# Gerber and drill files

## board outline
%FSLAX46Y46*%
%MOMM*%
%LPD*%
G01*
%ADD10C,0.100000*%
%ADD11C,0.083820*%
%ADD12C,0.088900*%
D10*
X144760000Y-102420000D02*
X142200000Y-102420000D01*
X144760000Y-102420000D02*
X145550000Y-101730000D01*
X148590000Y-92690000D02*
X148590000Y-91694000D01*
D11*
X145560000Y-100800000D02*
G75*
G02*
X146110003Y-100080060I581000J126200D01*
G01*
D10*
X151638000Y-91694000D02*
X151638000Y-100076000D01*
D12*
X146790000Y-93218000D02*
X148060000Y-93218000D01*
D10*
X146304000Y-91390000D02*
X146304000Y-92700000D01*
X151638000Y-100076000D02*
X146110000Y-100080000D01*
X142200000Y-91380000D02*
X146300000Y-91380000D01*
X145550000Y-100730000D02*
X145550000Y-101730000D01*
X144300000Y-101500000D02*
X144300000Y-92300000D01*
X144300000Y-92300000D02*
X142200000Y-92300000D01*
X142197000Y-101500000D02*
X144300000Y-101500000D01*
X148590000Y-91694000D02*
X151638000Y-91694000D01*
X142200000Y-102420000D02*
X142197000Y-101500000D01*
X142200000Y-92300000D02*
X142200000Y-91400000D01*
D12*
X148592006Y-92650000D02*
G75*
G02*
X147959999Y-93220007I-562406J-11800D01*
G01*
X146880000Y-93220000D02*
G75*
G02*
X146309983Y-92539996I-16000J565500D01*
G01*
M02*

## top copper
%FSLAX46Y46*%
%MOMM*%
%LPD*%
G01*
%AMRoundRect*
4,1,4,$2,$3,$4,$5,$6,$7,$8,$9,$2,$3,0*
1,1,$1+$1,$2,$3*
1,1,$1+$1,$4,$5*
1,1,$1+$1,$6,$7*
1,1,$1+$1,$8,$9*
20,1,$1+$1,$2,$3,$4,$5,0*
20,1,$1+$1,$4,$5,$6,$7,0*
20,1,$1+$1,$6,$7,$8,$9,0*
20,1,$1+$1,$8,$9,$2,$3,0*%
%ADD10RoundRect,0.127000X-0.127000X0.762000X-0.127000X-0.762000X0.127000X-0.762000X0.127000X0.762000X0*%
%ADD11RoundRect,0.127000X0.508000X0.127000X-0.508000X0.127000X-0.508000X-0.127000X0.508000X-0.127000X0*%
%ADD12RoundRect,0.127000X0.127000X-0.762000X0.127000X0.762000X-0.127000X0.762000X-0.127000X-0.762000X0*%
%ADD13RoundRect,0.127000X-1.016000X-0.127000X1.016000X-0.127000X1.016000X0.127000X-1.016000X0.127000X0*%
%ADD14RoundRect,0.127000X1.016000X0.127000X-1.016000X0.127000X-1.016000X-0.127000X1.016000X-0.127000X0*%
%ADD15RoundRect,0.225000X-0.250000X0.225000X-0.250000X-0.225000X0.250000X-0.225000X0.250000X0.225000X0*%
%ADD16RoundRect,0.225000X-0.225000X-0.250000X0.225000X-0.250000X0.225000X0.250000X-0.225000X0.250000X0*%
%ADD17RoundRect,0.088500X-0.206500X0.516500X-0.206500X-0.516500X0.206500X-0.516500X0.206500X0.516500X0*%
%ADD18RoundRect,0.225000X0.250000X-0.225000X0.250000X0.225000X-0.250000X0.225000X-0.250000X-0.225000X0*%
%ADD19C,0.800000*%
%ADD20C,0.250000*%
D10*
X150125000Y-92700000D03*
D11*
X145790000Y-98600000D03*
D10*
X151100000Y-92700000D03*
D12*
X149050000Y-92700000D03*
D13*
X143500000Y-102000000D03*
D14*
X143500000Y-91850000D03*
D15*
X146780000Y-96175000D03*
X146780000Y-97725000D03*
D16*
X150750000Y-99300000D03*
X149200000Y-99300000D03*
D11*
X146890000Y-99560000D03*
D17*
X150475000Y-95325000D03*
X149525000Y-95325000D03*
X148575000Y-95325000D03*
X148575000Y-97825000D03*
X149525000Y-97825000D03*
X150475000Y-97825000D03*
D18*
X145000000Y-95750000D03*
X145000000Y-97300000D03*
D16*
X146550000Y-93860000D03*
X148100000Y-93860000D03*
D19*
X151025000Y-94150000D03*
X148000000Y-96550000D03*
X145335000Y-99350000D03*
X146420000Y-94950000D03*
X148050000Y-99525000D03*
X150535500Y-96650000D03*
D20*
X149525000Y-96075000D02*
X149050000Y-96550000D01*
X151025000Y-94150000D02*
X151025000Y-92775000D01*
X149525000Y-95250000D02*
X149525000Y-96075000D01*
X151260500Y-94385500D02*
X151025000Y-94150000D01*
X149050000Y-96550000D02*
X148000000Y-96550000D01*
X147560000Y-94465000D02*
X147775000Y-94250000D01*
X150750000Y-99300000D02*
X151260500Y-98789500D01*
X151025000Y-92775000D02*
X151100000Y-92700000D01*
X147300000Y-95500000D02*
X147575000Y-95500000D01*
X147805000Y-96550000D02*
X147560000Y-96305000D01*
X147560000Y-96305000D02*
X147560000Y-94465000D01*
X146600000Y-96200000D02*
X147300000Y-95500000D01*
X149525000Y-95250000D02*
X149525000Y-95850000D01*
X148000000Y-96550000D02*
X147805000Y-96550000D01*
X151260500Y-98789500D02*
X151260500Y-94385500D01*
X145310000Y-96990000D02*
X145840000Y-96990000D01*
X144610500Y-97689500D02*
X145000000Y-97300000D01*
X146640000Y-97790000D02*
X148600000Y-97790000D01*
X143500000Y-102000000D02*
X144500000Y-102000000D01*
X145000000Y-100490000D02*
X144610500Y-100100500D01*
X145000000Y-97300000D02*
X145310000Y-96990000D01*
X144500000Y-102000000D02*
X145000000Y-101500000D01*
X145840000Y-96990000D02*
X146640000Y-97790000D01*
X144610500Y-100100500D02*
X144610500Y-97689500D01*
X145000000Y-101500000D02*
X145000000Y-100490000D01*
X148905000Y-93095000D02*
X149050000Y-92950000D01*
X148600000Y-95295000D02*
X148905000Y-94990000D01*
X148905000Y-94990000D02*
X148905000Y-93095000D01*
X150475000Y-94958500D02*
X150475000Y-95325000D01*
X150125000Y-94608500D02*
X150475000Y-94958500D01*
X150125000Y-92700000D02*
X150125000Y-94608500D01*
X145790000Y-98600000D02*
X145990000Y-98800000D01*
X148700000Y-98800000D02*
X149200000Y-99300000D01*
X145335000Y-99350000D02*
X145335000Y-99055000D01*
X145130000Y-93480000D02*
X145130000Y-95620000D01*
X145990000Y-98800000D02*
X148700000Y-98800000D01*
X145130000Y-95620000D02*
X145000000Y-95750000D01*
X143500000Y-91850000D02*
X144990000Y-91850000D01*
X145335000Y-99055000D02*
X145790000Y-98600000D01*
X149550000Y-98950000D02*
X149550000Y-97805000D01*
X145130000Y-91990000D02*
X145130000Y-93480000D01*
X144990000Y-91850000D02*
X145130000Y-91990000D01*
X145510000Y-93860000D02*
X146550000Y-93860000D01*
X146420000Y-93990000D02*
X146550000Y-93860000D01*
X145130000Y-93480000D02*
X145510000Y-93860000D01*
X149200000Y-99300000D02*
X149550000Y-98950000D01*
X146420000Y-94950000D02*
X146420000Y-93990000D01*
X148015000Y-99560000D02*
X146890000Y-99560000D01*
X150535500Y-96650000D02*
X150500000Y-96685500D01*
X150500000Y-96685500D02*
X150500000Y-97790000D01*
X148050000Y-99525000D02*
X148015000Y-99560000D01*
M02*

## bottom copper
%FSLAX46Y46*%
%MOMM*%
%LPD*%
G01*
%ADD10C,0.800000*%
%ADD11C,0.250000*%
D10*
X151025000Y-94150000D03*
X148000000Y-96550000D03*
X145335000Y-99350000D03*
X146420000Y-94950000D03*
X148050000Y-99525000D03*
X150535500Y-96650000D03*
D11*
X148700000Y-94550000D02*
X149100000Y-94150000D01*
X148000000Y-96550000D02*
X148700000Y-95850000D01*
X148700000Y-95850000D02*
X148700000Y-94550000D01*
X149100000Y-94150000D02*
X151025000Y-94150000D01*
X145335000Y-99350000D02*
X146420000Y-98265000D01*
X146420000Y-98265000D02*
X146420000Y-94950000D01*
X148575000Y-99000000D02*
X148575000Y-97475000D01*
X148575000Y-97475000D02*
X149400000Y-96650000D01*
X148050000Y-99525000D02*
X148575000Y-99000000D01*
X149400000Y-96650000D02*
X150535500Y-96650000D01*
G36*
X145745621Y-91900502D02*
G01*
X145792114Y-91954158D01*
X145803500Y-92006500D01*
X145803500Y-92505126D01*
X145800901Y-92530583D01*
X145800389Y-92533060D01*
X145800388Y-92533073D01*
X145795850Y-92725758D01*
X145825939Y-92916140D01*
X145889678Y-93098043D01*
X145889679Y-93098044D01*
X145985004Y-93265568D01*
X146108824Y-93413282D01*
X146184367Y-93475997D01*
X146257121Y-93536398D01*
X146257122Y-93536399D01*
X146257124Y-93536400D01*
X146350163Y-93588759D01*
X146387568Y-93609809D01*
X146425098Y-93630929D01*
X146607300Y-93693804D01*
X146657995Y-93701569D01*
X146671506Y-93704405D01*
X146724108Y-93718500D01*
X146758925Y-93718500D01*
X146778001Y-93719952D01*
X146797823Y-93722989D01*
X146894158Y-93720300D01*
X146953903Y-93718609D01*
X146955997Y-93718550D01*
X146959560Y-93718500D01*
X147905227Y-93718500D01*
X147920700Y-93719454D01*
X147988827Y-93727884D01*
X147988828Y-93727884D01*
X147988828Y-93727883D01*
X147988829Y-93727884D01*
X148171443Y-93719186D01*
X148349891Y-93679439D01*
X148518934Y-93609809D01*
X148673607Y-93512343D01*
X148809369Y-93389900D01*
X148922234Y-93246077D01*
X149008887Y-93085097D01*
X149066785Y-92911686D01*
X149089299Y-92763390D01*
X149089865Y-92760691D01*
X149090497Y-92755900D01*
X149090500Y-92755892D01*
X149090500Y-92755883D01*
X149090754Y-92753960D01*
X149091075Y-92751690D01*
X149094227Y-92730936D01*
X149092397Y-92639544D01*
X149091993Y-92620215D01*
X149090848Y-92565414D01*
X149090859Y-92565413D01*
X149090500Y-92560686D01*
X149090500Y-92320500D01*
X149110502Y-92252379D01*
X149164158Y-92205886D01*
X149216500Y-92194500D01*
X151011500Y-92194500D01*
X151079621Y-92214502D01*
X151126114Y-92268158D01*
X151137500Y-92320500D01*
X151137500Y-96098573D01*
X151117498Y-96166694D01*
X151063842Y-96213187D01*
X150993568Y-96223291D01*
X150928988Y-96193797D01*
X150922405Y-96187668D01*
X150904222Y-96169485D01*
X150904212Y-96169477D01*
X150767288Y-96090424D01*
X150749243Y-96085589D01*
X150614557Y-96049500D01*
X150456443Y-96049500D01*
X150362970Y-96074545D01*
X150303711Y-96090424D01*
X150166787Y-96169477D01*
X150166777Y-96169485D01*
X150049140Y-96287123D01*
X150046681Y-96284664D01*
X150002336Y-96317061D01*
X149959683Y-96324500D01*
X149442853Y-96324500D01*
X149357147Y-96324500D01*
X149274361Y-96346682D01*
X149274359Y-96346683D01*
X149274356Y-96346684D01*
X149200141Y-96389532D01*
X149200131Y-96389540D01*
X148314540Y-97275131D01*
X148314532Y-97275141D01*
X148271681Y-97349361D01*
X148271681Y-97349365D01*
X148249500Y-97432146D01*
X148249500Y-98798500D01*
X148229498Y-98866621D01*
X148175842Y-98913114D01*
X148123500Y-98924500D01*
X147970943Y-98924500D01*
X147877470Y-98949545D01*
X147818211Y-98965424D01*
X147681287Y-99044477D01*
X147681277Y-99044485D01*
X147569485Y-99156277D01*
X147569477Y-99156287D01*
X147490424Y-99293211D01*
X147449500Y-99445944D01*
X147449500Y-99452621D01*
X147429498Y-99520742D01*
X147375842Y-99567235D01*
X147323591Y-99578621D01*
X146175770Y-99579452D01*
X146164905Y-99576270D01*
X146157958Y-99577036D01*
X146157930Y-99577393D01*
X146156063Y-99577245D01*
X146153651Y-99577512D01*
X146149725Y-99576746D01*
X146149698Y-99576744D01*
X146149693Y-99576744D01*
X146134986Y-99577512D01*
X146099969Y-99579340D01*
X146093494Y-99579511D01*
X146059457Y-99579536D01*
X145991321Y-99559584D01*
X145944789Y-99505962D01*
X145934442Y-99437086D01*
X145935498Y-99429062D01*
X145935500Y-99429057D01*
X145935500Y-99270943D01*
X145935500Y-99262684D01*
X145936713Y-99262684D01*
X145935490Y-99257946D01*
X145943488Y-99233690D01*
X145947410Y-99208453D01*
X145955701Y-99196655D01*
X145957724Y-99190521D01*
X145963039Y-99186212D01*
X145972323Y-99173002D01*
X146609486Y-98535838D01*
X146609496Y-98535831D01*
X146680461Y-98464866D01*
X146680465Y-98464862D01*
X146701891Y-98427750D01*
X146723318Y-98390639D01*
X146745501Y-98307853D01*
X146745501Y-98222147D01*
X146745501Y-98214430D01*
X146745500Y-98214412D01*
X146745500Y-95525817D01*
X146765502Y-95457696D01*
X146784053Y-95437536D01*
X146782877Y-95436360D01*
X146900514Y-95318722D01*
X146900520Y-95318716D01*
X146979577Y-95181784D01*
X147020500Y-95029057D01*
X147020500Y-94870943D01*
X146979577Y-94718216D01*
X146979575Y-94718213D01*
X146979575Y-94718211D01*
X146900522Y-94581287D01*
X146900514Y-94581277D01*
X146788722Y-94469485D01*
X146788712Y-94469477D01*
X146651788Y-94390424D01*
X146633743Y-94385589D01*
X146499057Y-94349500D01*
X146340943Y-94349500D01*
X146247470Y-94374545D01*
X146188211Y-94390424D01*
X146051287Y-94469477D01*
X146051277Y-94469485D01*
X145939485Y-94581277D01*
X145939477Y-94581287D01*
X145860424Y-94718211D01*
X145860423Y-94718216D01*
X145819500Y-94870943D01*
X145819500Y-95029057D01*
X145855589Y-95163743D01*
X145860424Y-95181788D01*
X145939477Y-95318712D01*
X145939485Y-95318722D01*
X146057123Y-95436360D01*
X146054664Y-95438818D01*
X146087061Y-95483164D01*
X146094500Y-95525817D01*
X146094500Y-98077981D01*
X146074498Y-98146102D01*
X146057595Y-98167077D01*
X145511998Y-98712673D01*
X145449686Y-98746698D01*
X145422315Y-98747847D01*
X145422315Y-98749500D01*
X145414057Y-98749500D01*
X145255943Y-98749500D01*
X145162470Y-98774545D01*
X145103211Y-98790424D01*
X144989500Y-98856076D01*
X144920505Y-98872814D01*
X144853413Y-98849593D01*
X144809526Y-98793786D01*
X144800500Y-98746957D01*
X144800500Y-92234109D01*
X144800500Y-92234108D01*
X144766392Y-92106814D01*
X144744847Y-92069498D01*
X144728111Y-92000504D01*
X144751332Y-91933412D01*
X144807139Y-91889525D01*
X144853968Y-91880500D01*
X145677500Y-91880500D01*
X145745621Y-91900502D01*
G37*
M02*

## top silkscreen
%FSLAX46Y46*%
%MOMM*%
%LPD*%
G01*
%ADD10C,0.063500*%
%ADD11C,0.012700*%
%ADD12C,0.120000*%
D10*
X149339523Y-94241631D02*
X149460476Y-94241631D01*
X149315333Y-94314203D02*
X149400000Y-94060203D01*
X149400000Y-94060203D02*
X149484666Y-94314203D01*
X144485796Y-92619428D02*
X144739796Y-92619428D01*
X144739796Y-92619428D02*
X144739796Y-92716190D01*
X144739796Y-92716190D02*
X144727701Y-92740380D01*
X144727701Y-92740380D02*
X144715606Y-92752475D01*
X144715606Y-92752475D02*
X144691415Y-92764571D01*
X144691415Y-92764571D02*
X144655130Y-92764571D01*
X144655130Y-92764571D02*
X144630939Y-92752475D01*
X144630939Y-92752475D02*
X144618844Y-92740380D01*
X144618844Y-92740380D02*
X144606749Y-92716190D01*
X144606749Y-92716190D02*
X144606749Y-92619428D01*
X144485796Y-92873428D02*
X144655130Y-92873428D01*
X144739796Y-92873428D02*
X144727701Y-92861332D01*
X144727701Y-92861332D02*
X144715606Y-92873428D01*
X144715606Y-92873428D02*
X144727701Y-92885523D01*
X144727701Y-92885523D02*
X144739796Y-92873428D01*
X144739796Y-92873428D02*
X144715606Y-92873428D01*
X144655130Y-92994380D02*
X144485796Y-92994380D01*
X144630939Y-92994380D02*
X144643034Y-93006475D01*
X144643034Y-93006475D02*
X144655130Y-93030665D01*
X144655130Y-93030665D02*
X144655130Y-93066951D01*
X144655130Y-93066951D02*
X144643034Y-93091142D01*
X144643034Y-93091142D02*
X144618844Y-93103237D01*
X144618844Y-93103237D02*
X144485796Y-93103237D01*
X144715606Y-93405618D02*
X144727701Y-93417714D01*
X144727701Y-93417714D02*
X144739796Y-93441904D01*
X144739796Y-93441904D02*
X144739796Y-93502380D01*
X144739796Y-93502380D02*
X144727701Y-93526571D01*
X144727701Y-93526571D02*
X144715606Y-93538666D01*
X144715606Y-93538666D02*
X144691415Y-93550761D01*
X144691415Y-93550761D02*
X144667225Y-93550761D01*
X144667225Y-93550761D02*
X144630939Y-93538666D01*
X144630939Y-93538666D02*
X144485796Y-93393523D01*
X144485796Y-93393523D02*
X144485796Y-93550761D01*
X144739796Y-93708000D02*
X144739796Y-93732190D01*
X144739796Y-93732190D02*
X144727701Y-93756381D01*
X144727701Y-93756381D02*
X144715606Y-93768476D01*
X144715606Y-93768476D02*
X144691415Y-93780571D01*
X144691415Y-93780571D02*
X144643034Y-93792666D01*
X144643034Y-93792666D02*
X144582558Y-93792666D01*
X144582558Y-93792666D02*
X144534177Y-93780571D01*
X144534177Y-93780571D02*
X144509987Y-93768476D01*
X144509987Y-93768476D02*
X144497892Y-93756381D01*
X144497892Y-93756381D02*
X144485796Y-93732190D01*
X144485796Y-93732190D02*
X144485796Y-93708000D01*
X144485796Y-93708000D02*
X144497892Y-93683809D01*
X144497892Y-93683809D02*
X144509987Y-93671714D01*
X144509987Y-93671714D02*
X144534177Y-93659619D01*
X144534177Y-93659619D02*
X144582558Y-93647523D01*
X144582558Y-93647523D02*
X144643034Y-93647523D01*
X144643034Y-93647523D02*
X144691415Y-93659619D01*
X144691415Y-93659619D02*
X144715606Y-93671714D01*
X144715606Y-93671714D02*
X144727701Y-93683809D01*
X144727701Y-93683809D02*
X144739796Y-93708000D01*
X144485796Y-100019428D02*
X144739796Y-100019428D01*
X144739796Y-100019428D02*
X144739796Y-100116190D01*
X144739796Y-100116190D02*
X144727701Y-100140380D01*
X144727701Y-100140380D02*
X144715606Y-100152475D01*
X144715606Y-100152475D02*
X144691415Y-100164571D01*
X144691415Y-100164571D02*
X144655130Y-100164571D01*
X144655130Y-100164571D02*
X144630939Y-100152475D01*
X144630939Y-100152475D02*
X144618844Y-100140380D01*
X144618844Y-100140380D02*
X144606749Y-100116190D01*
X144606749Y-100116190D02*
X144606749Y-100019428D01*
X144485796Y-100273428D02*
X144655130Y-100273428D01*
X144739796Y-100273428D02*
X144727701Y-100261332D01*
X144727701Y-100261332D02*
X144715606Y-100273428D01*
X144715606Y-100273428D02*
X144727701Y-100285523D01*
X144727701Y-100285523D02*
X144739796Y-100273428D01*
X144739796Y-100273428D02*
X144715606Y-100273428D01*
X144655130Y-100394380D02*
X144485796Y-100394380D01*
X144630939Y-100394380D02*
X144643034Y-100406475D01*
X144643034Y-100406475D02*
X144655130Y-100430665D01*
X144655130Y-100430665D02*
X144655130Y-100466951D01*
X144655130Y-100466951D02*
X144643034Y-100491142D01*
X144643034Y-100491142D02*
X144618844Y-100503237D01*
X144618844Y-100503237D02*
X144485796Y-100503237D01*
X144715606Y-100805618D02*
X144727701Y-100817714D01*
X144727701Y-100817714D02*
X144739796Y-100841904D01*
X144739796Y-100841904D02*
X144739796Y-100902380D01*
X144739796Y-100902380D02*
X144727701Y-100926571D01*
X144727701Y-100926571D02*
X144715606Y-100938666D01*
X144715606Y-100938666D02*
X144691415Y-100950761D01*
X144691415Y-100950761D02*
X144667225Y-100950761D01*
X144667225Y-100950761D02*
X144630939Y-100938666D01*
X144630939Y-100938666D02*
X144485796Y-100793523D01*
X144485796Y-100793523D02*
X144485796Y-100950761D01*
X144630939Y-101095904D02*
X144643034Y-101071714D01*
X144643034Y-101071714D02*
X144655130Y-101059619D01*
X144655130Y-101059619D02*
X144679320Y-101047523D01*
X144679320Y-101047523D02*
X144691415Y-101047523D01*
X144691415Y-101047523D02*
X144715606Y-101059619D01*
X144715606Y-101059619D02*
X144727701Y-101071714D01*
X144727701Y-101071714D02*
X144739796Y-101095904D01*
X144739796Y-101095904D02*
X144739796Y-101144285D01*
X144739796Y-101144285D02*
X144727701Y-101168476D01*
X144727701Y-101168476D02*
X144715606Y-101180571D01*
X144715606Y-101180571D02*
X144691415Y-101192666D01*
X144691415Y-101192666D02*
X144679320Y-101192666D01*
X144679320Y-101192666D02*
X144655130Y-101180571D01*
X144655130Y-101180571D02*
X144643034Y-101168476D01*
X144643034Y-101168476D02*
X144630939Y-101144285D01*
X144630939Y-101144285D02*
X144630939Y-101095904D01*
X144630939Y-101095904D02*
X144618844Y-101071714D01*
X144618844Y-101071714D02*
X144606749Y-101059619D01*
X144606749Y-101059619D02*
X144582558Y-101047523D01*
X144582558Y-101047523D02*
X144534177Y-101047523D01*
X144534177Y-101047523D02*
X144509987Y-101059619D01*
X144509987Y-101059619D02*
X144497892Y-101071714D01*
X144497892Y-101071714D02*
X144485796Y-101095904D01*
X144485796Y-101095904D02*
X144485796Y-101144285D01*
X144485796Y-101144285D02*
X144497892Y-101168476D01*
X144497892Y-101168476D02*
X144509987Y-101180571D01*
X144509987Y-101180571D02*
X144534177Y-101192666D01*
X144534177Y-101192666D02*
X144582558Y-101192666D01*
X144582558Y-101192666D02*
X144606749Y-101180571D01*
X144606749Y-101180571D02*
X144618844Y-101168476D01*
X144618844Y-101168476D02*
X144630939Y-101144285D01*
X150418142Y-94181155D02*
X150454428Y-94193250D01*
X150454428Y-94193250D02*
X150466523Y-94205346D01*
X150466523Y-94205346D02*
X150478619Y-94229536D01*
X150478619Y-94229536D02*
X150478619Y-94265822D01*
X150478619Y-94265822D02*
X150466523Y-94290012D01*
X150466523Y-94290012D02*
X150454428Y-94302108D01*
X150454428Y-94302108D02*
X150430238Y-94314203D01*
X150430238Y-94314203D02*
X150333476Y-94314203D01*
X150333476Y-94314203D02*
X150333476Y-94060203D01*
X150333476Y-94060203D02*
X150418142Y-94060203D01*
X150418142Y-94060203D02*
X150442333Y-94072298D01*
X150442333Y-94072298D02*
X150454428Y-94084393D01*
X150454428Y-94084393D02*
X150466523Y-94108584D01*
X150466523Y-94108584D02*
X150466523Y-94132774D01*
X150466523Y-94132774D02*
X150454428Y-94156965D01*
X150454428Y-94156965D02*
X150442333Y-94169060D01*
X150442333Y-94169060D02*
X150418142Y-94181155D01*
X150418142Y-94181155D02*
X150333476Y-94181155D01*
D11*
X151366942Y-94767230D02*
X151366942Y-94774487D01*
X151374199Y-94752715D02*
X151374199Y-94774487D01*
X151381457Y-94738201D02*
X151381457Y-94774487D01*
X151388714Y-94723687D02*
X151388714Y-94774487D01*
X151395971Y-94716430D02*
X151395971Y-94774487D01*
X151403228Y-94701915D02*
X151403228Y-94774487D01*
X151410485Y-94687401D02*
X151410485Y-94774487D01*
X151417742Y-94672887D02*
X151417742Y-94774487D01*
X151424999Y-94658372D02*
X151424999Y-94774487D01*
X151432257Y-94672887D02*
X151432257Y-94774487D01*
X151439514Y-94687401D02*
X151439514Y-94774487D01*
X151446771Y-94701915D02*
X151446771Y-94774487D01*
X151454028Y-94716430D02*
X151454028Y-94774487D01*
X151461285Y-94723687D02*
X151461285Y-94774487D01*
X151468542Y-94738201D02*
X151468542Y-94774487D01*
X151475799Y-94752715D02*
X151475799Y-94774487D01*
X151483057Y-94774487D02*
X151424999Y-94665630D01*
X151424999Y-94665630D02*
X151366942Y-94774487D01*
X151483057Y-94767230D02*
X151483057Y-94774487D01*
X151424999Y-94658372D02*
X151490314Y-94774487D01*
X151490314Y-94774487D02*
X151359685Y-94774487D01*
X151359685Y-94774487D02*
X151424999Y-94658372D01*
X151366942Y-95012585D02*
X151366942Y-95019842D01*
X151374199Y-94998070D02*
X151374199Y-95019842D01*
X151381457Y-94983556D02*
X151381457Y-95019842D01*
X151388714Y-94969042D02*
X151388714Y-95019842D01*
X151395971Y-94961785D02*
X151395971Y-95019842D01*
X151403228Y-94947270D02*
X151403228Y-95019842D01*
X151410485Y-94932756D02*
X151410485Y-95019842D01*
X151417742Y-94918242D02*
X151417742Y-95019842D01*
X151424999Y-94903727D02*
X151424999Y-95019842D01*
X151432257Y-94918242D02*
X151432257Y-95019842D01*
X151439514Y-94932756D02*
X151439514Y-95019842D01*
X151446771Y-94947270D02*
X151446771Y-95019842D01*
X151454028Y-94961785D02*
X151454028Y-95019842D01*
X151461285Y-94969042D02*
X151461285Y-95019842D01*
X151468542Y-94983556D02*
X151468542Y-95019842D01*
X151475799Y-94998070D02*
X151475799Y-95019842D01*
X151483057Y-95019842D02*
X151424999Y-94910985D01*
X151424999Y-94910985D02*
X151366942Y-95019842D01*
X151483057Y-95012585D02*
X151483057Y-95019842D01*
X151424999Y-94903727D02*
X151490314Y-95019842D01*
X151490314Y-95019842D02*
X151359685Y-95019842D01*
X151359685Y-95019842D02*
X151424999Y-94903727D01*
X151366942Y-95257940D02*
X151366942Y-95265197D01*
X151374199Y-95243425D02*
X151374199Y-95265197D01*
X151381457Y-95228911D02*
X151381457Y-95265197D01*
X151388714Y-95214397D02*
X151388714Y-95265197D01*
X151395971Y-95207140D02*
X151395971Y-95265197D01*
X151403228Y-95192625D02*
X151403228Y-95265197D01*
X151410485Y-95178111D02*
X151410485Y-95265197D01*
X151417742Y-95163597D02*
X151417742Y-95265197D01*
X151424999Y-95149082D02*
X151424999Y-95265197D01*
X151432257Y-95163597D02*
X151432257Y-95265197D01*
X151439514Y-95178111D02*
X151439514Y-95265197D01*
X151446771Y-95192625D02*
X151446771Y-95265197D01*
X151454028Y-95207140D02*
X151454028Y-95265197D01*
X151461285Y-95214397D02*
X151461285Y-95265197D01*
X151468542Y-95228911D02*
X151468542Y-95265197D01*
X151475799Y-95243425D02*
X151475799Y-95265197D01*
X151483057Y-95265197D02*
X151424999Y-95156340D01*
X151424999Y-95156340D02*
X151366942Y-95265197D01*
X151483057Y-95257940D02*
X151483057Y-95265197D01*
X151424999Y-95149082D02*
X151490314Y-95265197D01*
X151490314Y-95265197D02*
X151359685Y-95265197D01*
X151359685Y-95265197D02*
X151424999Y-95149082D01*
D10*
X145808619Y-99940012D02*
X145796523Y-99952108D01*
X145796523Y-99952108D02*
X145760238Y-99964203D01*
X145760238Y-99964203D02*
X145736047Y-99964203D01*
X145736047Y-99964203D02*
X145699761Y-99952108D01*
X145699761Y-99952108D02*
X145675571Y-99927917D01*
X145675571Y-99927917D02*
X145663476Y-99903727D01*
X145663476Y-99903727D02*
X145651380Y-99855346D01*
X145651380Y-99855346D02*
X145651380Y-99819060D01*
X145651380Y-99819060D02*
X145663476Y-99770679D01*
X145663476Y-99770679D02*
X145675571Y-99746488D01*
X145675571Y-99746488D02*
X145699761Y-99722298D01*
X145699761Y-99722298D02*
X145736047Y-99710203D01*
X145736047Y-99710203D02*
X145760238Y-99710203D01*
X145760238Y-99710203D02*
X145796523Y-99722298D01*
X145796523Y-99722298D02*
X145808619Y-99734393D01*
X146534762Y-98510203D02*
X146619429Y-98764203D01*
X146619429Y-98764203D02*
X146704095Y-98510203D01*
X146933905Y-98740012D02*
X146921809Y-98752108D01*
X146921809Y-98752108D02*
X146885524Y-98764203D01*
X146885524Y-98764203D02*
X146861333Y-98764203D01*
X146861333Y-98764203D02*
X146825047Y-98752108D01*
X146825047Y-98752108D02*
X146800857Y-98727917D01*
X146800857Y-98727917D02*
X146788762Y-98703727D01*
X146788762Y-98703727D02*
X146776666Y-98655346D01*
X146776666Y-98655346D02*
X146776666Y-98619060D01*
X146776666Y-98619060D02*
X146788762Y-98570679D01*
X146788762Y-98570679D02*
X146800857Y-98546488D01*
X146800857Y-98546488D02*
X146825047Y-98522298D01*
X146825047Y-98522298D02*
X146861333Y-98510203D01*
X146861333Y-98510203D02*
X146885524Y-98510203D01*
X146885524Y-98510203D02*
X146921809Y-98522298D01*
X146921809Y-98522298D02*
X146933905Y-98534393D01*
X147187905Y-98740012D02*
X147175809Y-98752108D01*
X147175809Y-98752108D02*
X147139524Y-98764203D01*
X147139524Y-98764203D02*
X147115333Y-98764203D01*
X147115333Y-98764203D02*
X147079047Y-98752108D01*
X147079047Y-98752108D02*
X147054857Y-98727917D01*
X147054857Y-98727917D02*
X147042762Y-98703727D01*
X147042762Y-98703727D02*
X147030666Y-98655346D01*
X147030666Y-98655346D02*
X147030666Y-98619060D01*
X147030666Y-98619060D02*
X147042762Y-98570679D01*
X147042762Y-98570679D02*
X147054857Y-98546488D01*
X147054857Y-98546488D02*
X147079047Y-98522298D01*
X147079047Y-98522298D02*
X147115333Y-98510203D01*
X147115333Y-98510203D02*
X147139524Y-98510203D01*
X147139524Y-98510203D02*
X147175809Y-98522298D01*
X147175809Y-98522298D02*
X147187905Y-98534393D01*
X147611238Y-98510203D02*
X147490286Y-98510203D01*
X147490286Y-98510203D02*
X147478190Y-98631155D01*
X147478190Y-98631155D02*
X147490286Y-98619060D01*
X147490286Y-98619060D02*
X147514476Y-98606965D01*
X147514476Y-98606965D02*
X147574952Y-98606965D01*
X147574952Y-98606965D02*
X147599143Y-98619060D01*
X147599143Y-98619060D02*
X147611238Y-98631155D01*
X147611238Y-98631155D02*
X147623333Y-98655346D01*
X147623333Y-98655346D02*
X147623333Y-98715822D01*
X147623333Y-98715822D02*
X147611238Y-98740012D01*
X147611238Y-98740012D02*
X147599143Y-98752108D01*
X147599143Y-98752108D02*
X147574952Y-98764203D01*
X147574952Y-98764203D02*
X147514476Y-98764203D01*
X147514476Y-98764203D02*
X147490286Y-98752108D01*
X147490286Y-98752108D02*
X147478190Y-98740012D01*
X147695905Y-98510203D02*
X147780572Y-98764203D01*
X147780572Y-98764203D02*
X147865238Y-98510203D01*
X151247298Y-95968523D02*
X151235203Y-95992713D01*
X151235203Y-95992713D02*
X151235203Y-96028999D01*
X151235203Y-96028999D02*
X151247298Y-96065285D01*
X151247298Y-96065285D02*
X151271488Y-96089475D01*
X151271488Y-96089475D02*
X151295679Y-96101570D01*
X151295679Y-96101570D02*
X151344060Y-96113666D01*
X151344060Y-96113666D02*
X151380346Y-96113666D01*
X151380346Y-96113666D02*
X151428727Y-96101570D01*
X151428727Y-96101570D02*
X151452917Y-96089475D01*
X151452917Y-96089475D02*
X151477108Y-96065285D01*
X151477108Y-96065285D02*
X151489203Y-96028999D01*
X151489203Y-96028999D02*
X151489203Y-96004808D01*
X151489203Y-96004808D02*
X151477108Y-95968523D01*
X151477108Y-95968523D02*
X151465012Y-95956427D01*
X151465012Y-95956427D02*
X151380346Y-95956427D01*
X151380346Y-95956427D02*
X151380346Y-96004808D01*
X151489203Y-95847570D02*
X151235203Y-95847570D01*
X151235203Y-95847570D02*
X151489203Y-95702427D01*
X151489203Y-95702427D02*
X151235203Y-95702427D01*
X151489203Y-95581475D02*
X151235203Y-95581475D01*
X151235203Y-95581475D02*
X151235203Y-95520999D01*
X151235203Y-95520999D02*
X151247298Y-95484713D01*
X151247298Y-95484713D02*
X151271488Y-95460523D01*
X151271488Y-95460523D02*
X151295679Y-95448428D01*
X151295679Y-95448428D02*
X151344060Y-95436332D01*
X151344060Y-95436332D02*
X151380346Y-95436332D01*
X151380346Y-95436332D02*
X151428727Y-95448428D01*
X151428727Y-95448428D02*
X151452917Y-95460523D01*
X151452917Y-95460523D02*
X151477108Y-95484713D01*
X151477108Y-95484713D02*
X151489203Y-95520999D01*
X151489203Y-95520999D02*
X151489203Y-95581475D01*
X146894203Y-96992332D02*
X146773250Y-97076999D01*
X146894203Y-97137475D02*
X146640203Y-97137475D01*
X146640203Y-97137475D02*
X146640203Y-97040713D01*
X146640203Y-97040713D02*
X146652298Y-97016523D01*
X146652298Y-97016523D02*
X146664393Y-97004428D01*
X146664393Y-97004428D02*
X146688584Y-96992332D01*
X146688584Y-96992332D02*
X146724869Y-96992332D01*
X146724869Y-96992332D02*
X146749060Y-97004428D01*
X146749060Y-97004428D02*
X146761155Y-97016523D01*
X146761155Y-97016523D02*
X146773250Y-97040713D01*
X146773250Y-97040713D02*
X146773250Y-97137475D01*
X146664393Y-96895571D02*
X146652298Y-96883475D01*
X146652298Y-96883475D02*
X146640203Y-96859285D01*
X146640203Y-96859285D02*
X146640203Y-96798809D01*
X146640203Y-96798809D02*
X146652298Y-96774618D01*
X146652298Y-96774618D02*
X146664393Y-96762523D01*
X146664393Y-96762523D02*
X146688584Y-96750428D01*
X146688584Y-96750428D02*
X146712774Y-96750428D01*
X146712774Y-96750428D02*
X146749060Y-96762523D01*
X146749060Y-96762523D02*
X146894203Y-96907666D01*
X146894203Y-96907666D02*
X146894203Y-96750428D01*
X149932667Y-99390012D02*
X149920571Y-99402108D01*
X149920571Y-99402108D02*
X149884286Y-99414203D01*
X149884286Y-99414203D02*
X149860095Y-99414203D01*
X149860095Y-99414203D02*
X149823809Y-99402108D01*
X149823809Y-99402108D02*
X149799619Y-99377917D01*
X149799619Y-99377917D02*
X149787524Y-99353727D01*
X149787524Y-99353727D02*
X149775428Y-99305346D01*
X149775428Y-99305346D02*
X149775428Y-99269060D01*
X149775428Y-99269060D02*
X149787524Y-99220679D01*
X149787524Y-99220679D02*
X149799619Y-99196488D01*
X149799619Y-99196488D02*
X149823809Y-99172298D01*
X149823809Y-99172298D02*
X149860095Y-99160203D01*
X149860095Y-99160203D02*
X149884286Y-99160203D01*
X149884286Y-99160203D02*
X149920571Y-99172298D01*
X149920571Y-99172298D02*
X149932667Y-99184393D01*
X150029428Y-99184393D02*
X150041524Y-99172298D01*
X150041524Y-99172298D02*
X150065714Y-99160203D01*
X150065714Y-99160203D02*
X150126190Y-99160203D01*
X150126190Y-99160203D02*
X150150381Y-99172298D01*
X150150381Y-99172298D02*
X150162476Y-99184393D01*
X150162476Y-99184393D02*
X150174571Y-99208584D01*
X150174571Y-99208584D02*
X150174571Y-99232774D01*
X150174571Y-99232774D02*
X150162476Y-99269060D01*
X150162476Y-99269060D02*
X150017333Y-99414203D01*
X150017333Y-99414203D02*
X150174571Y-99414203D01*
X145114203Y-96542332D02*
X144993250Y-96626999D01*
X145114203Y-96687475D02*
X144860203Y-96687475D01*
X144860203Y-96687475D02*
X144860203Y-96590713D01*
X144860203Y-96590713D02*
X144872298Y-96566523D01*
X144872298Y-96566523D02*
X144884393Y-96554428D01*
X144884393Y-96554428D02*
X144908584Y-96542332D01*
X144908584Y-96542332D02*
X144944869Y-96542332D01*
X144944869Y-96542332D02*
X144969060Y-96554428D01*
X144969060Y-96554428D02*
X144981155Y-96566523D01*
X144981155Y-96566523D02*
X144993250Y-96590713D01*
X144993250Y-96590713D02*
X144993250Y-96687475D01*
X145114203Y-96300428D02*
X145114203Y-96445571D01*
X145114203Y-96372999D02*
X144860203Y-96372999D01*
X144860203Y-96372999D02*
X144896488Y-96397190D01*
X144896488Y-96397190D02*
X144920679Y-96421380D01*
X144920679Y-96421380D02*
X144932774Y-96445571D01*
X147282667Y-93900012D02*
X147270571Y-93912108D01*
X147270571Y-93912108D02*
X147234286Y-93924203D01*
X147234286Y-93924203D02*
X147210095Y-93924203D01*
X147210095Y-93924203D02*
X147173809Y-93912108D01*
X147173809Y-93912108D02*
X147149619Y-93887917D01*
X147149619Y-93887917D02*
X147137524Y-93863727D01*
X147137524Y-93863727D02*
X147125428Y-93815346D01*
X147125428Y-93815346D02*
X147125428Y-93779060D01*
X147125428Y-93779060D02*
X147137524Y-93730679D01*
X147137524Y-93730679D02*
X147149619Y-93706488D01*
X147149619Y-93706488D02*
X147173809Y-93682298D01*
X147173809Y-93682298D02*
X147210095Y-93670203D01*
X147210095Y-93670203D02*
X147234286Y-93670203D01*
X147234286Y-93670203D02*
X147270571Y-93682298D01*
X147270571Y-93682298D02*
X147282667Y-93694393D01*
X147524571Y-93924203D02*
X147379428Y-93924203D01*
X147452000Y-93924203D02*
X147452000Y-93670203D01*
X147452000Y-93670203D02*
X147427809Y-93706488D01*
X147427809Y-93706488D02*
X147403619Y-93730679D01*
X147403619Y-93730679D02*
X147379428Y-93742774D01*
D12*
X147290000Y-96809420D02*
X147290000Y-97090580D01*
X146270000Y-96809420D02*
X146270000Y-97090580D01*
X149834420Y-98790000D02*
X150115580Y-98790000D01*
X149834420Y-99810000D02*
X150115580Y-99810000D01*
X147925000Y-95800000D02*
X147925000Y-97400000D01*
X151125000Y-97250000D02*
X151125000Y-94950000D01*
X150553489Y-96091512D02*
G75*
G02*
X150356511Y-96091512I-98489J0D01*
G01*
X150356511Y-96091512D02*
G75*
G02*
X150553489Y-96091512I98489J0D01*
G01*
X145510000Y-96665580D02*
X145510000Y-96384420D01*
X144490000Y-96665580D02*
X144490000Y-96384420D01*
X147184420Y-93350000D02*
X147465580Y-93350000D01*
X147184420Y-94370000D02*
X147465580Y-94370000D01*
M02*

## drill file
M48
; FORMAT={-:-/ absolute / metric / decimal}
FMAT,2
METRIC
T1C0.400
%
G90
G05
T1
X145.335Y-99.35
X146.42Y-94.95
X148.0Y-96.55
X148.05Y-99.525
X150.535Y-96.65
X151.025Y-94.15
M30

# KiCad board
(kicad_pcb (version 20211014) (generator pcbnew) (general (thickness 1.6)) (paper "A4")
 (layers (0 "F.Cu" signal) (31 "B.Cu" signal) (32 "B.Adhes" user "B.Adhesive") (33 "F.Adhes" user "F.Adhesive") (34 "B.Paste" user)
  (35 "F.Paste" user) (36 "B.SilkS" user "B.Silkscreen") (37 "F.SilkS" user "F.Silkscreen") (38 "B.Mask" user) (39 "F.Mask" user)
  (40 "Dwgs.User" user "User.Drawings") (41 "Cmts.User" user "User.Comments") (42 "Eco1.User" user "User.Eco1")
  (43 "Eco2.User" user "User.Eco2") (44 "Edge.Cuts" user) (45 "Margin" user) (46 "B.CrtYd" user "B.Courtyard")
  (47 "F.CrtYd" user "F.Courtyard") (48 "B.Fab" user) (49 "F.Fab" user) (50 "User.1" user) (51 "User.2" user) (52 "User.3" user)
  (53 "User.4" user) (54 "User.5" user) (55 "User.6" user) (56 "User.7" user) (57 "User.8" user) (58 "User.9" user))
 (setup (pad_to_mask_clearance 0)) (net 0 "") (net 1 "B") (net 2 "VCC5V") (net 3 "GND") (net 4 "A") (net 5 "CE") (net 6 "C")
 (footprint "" (layer "F.Cu") (at 150.125 92.7 90)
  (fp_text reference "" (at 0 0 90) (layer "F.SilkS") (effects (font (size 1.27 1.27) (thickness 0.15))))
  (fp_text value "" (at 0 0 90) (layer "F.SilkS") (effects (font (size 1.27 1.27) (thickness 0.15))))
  (pad "10" smd roundrect (at 0 0 270) (size 1.778 0.508) (layers "F.Cu" "F.Paste" "F.Mask") (roundrect_rratio 0.25) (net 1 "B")))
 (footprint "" (layer "F.Cu") (at 145.79 98.6 -90)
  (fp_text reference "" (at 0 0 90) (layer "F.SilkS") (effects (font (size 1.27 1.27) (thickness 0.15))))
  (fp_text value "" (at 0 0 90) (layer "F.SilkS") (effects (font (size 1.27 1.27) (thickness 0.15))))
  (pad "B" smd roundrect (at 0 0 180) (size 1.27 0.508) (layers "F.Cu" "F.Paste" "F.Mask") (roundrect_rratio 0.25) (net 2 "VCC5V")))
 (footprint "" (layer "F.Cu") (at 151.1 92.7 90)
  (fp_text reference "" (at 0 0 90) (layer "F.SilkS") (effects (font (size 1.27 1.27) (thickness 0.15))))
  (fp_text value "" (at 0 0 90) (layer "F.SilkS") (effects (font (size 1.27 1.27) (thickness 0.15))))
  (pad "9" smd roundrect (at 0 0 270) (size 1.778 0.508) (layers "F.Cu" "F.Paste" "F.Mask") (roundrect_rratio 0.25) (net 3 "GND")))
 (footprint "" (layer "F.Cu") (at 149.05 92.7 -90)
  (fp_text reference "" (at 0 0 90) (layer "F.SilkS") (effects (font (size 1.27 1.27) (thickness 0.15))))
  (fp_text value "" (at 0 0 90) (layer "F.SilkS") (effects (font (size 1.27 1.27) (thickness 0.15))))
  (pad "11" smd roundrect (at 0 0 90) (size 1.778 0.508) (layers "F.Cu" "F.Paste" "F.Mask") (roundrect_rratio 0.25) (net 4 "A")))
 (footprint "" (layer "F.Cu") (at 143.5 102)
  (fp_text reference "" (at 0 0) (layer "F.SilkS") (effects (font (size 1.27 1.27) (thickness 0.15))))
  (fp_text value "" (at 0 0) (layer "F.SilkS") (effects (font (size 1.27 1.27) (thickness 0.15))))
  (pad "4" smd roundrect (at 0 0) (size 2.286 0.508) (layers "F.Cu" "F.Paste" "F.Mask") (roundrect_rratio 0.25) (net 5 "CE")))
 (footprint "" (layer "F.Cu") (at 143.5 91.85 180)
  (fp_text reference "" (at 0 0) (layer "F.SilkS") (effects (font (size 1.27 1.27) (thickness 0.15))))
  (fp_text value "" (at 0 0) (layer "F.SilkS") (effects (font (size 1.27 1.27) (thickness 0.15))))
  (pad "1" smd roundrect (at 0 0 180) (size 2.286 0.508) (layers "F.Cu" "F.Paste" "F.Mask") (roundrect_rratio 0.25) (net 2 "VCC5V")))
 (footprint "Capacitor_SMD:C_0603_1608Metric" (layer "F.Cu") (at 146.78 96.95 -90)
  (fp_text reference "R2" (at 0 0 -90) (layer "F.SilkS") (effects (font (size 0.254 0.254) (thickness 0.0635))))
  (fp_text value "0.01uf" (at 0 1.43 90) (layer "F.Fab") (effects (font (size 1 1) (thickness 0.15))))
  (fp_line (start -0.14058 -0.51) (end 0.14058 -0.51) (layer "F.SilkS") (width 0.12))
  (fp_line (start -0.14058 0.51) (end 0.14058 0.51) (layer "F.SilkS") (width 0.12))
  (pad "5" smd roundrect (at -0.775 0 270) (size 0.9 0.95) (layers "F.Cu" "F.Paste" "F.Mask") (roundrect_rratio 0.25) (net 3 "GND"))
  (pad "6" smd roundrect (at 0.775 0 270) (size 0.9 0.95) (layers "F.Cu" "F.Paste" "F.Mask") (roundrect_rratio 0.25) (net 5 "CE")))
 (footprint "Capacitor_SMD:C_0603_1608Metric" (layer "F.Cu") (at 149.975 99.3)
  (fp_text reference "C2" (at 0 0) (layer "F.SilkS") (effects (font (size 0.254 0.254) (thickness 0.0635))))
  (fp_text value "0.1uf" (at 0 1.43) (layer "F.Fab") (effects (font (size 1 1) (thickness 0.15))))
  (fp_line (start -0.14058 -0.51) (end 0.14058 -0.51) (layer "F.SilkS") (width 0.12))
  (fp_line (start -0.14058 0.51) (end 0.14058 0.51) (layer "F.SilkS") (width 0.12))
  (pad "7" smd roundrect (at 0.775 0) (size 0.9 0.95) (layers "F.Cu" "F.Paste" "F.Mask") (roundrect_rratio 0.25) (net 3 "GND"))
  (pad "8" smd roundrect (at -0.775 0) (size 0.9 0.95) (layers "F.Cu" "F.Paste" "F.Mask") (roundrect_rratio 0.25) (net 2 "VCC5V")))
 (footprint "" (layer "F.Cu") (at 146.89 99.56)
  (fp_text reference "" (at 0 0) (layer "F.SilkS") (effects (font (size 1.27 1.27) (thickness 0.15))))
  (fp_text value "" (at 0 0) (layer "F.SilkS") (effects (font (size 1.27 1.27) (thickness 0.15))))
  (pad "B" smd roundrect (at 0 0 180) (size 1.27 0.508) (layers "F.Cu" "F.Paste" "F.Mask") (roundrect_rratio 0.25) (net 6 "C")))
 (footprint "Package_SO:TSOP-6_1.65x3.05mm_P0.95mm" (layer "F.Cu") (at 149.525 96.45 -90)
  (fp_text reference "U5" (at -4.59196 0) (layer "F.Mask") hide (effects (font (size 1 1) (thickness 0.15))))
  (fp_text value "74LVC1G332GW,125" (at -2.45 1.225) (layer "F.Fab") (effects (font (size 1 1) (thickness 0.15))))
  (fp_line (start -0.65 1.6) (end 0.95 1.6) (layer "F.SilkS") (width 0.12))
  (fp_line (start 0.8 -1.6) (end -1.5 -1.6) (layer "F.SilkS") (width 0.12))
  (fp_circle (center -0.358488 -0.93) (end -0.268488 -0.89) (layer "F.SilkS") (width 0.12) (fill none))
  (pad "1" smd roundrect (at -1.125 -0.95 270) (size 1.21 0.59) (layers "F.Cu" "F.Paste" "F.Mask") (roundrect_rratio 0.15) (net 1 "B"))
  (pad "2" smd roundrect (at -1.125 0 270) (size 1.21 0.59) (layers "F.Cu" "F.Paste" "F.Mask") (roundrect_rratio 0.15) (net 3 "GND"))
  (pad "3" smd roundrect (at -1.125 0.95 270) (size 1.21 0.59) (layers "F.Cu" "F.Paste" "F.Mask") (roundrect_rratio 0.15) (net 4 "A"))
  (pad "4" smd roundrect (at 1.375 0.95 270) (size 1.21 0.59) (layers "F.Cu" "F.Paste" "F.Mask") (roundrect_rratio 0.15) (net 5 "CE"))
  (pad "5" smd roundrect (at 1.375 0 270) (size 1.21 0.59) (layers "F.Cu" "F.Paste" "F.Mask") (roundrect_rratio 0.15) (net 2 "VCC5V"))
  (pad "6" smd roundrect (at 1.375 -0.95 270) (size 1.21 0.59) (layers "F.Cu" "F.Paste" "F.Mask") (roundrect_rratio 0.15) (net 6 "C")))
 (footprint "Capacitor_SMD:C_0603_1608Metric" (layer "F.Cu") (at 145 96.525 90)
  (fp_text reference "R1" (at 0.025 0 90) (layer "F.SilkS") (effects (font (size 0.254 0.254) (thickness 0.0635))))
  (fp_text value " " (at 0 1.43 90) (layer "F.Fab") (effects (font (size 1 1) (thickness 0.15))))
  (fp_line (start -0.14058 0.51) (end 0.14058 0.51) (layer "F.SilkS") (width 0.12))
  (fp_line (start -0.14058 -0.51) (end 0.14058 -0.51) (layer "F.SilkS") (width 0.12))
  (pad "2" smd roundrect (at 0.775 0 90) (size 0.9 0.95) (layers "F.Cu" "F.Paste" "F.Mask") (roundrect_rratio 0.25) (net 2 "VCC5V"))
  (pad "3" smd roundrect (at -0.775 0 90) (size 0.9 0.95) (layers "F.Cu" "F.Paste" "F.Mask") (roundrect_rratio 0.25) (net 5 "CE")))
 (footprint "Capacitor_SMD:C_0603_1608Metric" (layer "F.Cu") (at 147.325 93.86)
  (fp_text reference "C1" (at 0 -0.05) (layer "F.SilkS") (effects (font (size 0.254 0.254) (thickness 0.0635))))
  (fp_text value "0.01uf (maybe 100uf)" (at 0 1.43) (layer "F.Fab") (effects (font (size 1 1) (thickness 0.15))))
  (fp_line (start -0.14058 -0.51) (end 0.14058 -0.51) (layer "F.SilkS") (width 0.12))
  (fp_line (start -0.14058 0.51) (end 0.14058 0.51) (layer "F.SilkS") (width 0.12))
  (pad "5" smd roundrect (at -0.775 0) (size 0.9 0.95) (layers "F.Cu" "F.Paste" "F.Mask") (roundrect_rratio 0.25) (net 2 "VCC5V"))
  (pad "6" smd roundrect (at 0.775 0) (size 0.9 0.95) (layers "F.Cu" "F.Paste" "F.Mask") (roundrect_rratio 0.25) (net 3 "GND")))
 (gr_line (start 144.76 102.42) (end 142.2 102.42) (layer "Edge.Cuts") (width 0.1))
 (gr_line (start 144.76 102.42) (end 145.55 101.73) (layer "Edge.Cuts") (width 0.1))
 (gr_line (start 148.59 92.69) (end 148.59 91.694) (layer "Edge.Cuts") (width 0.1))
 (gr_arc (start 145.56 100.8) (mid 145.667107 100.314693) (end 146.11 100.08) (layer "Edge.Cuts") (width 0.08382))
 (gr_line (start 151.638 91.694) (end 151.638 100.076) (layer "Edge.Cuts") (width 0.1))
 (gr_line (start 146.79 93.218) (end 148.06 93.218) (layer "Edge.Cuts") (width 0.0889))
 (gr_line (start 146.304 91.39) (end 146.304 92.7) (layer "Edge.Cuts") (width 0.1))
 (gr_line (start 151.638 100.076) (end 146.11 100.08) (layer "Edge.Cuts") (width 0.1))
 (gr_line (start 142.2 91.38) (end 146.3 91.38) (layer "Edge.Cuts") (width 0.1))
 (gr_line (start 145.55 100.73) (end 145.55 101.73) (layer "Edge.Cuts") (width 0.1))
 (gr_line (start 144.3 101.5) (end 144.3 92.3) (layer "Edge.Cuts") (width 0.1))
 (gr_line (start 144.3 92.3) (end 142.2 92.3) (layer "Edge.Cuts") (width 0.1))
 (gr_line (start 142.197 101.5) (end 144.3 101.5) (layer "Edge.Cuts") (width 0.1))
 (gr_line (start 148.59 91.694) (end 151.638 91.694) (layer "Edge.Cuts") (width 0.1))
 (gr_line (start 142.2 102.42) (end 142.197 101.5) (layer "Edge.Cuts") (width 0.1))
 (gr_line (start 142.2 92.3) (end 142.2 91.4) (layer "Edge.Cuts") (width 0.1))
 (gr_arc (start 148.592006 92.65) (mid 148.406336 93.079511) (end 147.96 93.22) (layer "Edge.Cuts") (width 0.0889))
 (gr_arc (start 146.88 93.22) (mid 146.430454 93.017928) (end 146.31 92.54) (layer "Edge.Cuts") (width 0.0889))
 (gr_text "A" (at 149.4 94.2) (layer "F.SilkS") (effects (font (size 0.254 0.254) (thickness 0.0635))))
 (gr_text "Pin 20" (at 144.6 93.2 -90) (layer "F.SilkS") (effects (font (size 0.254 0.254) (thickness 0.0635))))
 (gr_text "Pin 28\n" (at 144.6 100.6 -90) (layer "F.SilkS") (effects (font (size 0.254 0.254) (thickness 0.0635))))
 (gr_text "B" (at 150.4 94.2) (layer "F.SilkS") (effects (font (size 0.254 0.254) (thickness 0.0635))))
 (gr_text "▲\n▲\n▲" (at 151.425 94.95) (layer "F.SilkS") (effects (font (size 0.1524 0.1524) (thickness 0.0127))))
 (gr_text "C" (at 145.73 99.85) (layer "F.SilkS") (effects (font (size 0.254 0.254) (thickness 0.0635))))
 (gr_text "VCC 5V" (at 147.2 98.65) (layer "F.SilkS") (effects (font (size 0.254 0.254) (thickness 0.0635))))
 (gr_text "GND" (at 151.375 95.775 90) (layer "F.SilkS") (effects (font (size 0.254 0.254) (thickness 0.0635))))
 (segment (start 149.525 96.075) (end 149.05 96.55) (width 0.25) (layer "F.Cu") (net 3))
 (segment (start 151.025 94.15) (end 151.025 92.775) (width 0.25) (layer "F.Cu") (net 3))
 (segment (start 149.525 95.25) (end 149.525 96.075) (width 0.25) (layer "F.Cu") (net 3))
 (segment (start 151.2605 94.3855) (end 151.025 94.15) (width 0.25) (layer "F.Cu") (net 3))
 (segment (start 149.05 96.55) (end 148 96.55) (width 0.25) (layer "F.Cu") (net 3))
 (segment (start 147.56 94.465) (end 147.775 94.25) (width 0.25) (layer "F.Cu") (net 3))
 (segment (start 150.75 99.3) (end 151.2605 98.7895) (width 0.25) (layer "F.Cu") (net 3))
 (segment (start 151.025 92.775) (end 151.1 92.7) (width 0.25) (layer "F.Cu") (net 3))
 (segment (start 147.3 95.5) (end 147.575 95.5) (width 0.25) (layer "F.Cu") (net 3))
 (segment (start 147.805 96.55) (end 147.56 96.305) (width 0.25) (layer "F.Cu") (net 3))
 (segment (start 147.56 96.305) (end 147.56 94.465) (width 0.25) (layer "F.Cu") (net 3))
 (segment (start 146.6 96.2) (end 147.3 95.5) (width 0.25) (layer "F.Cu") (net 3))
 (segment (start 149.525 95.25) (end 149.525 95.85) (width 0.25) (layer "F.Cu") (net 3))
 (segment (start 148 96.55) (end 147.805 96.55) (width 0.25) (layer "F.Cu") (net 3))
 (segment (start 151.2605 98.7895) (end 151.2605 94.3855) (width 0.25) (layer "F.Cu") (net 3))
 (via (at 151.025 94.15) (size 0.8) (drill 0.4) (layers "F.Cu" "B.Cu") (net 3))
 (via (at 148 96.55) (size 0.8) (drill 0.4) (layers "F.Cu" "B.Cu") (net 3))
 (segment (start 148.7 94.55) (end 149.1 94.15) (width 0.25) (layer "B.Cu") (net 3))
 (segment (start 148 96.55) (end 148.7 95.85) (width 0.25) (layer "B.Cu") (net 3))
 (segment (start 148.7 95.85) (end 148.7 94.55) (width 0.25) (layer "B.Cu") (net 3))
 (segment (start 149.1 94.15) (end 151.025 94.15) (width 0.25) (layer "B.Cu") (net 3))
 (segment (start 145.31 96.99) (end 145.84 96.99) (width 0.25) (layer "F.Cu") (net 5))
 (segment (start 144.6105 97.6895) (end 145 97.3) (width 0.25) (layer "F.Cu") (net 5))
 (segment (start 146.64 97.79) (end 148.6 97.79) (width 0.25) (layer "F.Cu") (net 5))
 (segment (start 143.5 102) (end 144.5 102) (width 0.25) (layer "F.Cu") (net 5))
 (segment (start 145 100.49) (end 144.6105 100.1005) (width 0.25) (layer "F.Cu") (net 5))
 (segment (start 145 97.3) (end 145.31 96.99) (width 0.25) (layer "F.Cu") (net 5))
 (segment (start 144.5 102) (end 145 101.5) (width 0.25) (layer "F.Cu") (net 5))
 (segment (start 145.84 96.99) (end 146.64 97.79) (width 0.25) (layer "F.Cu") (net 5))
 (segment (start 144.6105 100.1005) (end 144.6105 97.6895) (width 0.25) (layer "F.Cu") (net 5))
 (segment (start 145 101.5) (end 145 100.49) (width 0.25) (layer "F.Cu") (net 5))
 (segment (start 148.905 93.095) (end 149.05 92.95) (width 0.25) (layer "F.Cu") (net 4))
 (segment (start 148.6 95.295) (end 148.905 94.99) (width 0.25) (layer "F.Cu") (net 4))
 (segment (start 148.905 94.99) (end 148.905 93.095) (width 0.25) (layer "F.Cu") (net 4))
 (segment (start 150.475 94.9585) (end 150.475 95.325) (width 0.25) (layer "F.Cu") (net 1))
 (segment (start 150.125 94.6085) (end 150.475 94.9585) (width 0.25) (layer "F.Cu") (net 1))
 (segment (start 150.125 92.7) (end 150.125 94.6085) (width 0.25) (layer "F.Cu") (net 1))
 (segment (start 145.79 98.6) (end 145.99 98.8) (width 0.25) (layer "F.Cu") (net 2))
 (segment (start 148.7 98.8) (end 149.2 99.3) (width 0.25) (layer "F.Cu") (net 2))
 (segment (start 145.335 99.35) (end 145.335 99.055) (width 0.25) (layer "F.Cu") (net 2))
 (segment (start 145.13 93.48) (end 145.13 95.62) (width 0.25) (layer "F.Cu") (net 2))
 (segment (start 145.99 98.8) (end 148.7 98.8) (width 0.25) (layer "F.Cu") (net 2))
 (segment (start 145.13 95.62) (end 145 95.75) (width 0.25) (layer "F.Cu") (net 2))
 (segment (start 143.5 91.85) (end 144.99 91.85) (width 0.25) (layer "F.Cu") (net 2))
 (segment (start 145.335 99.055) (end 145.79 98.6) (width 0.25) (layer "F.Cu") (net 2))
 (segment (start 149.55 98.95) (end 149.55 97.805) (width 0.25) (layer "F.Cu") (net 2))
 (segment (start 145.13 91.99) (end 145.13 93.48) (width 0.25) (layer "F.Cu") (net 2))
 (segment (start 144.99 91.85) (end 145.13 91.99) (width 0.25) (layer "F.Cu") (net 2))
 (segment (start 145.51 93.86) (end 146.55 93.86) (width 0.25) (layer "F.Cu") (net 2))
 (segment (start 146.42 93.99) (end 146.55 93.86) (width 0.25) (layer "F.Cu") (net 2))
 (segment (start 145.13 93.48) (end 145.51 93.86) (width 0.25) (layer "F.Cu") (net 2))
 (segment (start 149.2 99.3) (end 149.55 98.95) (width 0.25) (layer "F.Cu") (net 2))
 (segment (start 146.42 94.95) (end 146.42 93.99) (width 0.25) (layer "F.Cu") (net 2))
 (via (at 145.335 99.35) (size 0.8) (drill 0.4) (layers "F.Cu" "B.Cu") (free) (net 2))
 (via (at 146.42 94.95) (size 0.8) (drill 0.4) (layers "F.Cu" "B.Cu") (free) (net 2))
 (segment (start 145.335 99.35) (end 146.42 98.265) (width 0.25) (layer "B.Cu") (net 2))
 (segment (start 146.42 98.265) (end 146.42 94.95) (width 0.25) (layer "B.Cu") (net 2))
 (segment (start 148.015 99.56) (end 146.89 99.56) (width 0.25) (layer "F.Cu") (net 6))
 (segment (start 150.5355 96.65) (end 150.5 96.6855) (width 0.25) (layer "F.Cu") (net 6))
 (segment (start 150.5 96.6855) (end 150.5 97.79) (width 0.25) (layer "F.Cu") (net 6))
 (segment (start 148.05 99.525) (end 148.015 99.56) (width 0.25) (layer "F.Cu") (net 6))
 (via (at 148.05 99.525) (size 0.8) (drill 0.4) (layers "F.Cu" "B.Cu") (free) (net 6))
 (via (at 150.5355 96.65) (size 0.8) (drill 0.4) (layers "F.Cu" "B.Cu") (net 6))
 (segment (start 148.575 99) (end 148.575 97.475) (width 0.25) (layer "B.Cu") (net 6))
 (segment (start 148.575 97.475) (end 149.4 96.65) (width 0.25) (layer "B.Cu") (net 6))
 (segment (start 148.05 99.525) (end 148.575 99) (width 0.25) (layer "B.Cu") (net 6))
 (segment (start 149.4 96.65) (end 150.5355 96.65) (width 0.25) (layer "B.Cu") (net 6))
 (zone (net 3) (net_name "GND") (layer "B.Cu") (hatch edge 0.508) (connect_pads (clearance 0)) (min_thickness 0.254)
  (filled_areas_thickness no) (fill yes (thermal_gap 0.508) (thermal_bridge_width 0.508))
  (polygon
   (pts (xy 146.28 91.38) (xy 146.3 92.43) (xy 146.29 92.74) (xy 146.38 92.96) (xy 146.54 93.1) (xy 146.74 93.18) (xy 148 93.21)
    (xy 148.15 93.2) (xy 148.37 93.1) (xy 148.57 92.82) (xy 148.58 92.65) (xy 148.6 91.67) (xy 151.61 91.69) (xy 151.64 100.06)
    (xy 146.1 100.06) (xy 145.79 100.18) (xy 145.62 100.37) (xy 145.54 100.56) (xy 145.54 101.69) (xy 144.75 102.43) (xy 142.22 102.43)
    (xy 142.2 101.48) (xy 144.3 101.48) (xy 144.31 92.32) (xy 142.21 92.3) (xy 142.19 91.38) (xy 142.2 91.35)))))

